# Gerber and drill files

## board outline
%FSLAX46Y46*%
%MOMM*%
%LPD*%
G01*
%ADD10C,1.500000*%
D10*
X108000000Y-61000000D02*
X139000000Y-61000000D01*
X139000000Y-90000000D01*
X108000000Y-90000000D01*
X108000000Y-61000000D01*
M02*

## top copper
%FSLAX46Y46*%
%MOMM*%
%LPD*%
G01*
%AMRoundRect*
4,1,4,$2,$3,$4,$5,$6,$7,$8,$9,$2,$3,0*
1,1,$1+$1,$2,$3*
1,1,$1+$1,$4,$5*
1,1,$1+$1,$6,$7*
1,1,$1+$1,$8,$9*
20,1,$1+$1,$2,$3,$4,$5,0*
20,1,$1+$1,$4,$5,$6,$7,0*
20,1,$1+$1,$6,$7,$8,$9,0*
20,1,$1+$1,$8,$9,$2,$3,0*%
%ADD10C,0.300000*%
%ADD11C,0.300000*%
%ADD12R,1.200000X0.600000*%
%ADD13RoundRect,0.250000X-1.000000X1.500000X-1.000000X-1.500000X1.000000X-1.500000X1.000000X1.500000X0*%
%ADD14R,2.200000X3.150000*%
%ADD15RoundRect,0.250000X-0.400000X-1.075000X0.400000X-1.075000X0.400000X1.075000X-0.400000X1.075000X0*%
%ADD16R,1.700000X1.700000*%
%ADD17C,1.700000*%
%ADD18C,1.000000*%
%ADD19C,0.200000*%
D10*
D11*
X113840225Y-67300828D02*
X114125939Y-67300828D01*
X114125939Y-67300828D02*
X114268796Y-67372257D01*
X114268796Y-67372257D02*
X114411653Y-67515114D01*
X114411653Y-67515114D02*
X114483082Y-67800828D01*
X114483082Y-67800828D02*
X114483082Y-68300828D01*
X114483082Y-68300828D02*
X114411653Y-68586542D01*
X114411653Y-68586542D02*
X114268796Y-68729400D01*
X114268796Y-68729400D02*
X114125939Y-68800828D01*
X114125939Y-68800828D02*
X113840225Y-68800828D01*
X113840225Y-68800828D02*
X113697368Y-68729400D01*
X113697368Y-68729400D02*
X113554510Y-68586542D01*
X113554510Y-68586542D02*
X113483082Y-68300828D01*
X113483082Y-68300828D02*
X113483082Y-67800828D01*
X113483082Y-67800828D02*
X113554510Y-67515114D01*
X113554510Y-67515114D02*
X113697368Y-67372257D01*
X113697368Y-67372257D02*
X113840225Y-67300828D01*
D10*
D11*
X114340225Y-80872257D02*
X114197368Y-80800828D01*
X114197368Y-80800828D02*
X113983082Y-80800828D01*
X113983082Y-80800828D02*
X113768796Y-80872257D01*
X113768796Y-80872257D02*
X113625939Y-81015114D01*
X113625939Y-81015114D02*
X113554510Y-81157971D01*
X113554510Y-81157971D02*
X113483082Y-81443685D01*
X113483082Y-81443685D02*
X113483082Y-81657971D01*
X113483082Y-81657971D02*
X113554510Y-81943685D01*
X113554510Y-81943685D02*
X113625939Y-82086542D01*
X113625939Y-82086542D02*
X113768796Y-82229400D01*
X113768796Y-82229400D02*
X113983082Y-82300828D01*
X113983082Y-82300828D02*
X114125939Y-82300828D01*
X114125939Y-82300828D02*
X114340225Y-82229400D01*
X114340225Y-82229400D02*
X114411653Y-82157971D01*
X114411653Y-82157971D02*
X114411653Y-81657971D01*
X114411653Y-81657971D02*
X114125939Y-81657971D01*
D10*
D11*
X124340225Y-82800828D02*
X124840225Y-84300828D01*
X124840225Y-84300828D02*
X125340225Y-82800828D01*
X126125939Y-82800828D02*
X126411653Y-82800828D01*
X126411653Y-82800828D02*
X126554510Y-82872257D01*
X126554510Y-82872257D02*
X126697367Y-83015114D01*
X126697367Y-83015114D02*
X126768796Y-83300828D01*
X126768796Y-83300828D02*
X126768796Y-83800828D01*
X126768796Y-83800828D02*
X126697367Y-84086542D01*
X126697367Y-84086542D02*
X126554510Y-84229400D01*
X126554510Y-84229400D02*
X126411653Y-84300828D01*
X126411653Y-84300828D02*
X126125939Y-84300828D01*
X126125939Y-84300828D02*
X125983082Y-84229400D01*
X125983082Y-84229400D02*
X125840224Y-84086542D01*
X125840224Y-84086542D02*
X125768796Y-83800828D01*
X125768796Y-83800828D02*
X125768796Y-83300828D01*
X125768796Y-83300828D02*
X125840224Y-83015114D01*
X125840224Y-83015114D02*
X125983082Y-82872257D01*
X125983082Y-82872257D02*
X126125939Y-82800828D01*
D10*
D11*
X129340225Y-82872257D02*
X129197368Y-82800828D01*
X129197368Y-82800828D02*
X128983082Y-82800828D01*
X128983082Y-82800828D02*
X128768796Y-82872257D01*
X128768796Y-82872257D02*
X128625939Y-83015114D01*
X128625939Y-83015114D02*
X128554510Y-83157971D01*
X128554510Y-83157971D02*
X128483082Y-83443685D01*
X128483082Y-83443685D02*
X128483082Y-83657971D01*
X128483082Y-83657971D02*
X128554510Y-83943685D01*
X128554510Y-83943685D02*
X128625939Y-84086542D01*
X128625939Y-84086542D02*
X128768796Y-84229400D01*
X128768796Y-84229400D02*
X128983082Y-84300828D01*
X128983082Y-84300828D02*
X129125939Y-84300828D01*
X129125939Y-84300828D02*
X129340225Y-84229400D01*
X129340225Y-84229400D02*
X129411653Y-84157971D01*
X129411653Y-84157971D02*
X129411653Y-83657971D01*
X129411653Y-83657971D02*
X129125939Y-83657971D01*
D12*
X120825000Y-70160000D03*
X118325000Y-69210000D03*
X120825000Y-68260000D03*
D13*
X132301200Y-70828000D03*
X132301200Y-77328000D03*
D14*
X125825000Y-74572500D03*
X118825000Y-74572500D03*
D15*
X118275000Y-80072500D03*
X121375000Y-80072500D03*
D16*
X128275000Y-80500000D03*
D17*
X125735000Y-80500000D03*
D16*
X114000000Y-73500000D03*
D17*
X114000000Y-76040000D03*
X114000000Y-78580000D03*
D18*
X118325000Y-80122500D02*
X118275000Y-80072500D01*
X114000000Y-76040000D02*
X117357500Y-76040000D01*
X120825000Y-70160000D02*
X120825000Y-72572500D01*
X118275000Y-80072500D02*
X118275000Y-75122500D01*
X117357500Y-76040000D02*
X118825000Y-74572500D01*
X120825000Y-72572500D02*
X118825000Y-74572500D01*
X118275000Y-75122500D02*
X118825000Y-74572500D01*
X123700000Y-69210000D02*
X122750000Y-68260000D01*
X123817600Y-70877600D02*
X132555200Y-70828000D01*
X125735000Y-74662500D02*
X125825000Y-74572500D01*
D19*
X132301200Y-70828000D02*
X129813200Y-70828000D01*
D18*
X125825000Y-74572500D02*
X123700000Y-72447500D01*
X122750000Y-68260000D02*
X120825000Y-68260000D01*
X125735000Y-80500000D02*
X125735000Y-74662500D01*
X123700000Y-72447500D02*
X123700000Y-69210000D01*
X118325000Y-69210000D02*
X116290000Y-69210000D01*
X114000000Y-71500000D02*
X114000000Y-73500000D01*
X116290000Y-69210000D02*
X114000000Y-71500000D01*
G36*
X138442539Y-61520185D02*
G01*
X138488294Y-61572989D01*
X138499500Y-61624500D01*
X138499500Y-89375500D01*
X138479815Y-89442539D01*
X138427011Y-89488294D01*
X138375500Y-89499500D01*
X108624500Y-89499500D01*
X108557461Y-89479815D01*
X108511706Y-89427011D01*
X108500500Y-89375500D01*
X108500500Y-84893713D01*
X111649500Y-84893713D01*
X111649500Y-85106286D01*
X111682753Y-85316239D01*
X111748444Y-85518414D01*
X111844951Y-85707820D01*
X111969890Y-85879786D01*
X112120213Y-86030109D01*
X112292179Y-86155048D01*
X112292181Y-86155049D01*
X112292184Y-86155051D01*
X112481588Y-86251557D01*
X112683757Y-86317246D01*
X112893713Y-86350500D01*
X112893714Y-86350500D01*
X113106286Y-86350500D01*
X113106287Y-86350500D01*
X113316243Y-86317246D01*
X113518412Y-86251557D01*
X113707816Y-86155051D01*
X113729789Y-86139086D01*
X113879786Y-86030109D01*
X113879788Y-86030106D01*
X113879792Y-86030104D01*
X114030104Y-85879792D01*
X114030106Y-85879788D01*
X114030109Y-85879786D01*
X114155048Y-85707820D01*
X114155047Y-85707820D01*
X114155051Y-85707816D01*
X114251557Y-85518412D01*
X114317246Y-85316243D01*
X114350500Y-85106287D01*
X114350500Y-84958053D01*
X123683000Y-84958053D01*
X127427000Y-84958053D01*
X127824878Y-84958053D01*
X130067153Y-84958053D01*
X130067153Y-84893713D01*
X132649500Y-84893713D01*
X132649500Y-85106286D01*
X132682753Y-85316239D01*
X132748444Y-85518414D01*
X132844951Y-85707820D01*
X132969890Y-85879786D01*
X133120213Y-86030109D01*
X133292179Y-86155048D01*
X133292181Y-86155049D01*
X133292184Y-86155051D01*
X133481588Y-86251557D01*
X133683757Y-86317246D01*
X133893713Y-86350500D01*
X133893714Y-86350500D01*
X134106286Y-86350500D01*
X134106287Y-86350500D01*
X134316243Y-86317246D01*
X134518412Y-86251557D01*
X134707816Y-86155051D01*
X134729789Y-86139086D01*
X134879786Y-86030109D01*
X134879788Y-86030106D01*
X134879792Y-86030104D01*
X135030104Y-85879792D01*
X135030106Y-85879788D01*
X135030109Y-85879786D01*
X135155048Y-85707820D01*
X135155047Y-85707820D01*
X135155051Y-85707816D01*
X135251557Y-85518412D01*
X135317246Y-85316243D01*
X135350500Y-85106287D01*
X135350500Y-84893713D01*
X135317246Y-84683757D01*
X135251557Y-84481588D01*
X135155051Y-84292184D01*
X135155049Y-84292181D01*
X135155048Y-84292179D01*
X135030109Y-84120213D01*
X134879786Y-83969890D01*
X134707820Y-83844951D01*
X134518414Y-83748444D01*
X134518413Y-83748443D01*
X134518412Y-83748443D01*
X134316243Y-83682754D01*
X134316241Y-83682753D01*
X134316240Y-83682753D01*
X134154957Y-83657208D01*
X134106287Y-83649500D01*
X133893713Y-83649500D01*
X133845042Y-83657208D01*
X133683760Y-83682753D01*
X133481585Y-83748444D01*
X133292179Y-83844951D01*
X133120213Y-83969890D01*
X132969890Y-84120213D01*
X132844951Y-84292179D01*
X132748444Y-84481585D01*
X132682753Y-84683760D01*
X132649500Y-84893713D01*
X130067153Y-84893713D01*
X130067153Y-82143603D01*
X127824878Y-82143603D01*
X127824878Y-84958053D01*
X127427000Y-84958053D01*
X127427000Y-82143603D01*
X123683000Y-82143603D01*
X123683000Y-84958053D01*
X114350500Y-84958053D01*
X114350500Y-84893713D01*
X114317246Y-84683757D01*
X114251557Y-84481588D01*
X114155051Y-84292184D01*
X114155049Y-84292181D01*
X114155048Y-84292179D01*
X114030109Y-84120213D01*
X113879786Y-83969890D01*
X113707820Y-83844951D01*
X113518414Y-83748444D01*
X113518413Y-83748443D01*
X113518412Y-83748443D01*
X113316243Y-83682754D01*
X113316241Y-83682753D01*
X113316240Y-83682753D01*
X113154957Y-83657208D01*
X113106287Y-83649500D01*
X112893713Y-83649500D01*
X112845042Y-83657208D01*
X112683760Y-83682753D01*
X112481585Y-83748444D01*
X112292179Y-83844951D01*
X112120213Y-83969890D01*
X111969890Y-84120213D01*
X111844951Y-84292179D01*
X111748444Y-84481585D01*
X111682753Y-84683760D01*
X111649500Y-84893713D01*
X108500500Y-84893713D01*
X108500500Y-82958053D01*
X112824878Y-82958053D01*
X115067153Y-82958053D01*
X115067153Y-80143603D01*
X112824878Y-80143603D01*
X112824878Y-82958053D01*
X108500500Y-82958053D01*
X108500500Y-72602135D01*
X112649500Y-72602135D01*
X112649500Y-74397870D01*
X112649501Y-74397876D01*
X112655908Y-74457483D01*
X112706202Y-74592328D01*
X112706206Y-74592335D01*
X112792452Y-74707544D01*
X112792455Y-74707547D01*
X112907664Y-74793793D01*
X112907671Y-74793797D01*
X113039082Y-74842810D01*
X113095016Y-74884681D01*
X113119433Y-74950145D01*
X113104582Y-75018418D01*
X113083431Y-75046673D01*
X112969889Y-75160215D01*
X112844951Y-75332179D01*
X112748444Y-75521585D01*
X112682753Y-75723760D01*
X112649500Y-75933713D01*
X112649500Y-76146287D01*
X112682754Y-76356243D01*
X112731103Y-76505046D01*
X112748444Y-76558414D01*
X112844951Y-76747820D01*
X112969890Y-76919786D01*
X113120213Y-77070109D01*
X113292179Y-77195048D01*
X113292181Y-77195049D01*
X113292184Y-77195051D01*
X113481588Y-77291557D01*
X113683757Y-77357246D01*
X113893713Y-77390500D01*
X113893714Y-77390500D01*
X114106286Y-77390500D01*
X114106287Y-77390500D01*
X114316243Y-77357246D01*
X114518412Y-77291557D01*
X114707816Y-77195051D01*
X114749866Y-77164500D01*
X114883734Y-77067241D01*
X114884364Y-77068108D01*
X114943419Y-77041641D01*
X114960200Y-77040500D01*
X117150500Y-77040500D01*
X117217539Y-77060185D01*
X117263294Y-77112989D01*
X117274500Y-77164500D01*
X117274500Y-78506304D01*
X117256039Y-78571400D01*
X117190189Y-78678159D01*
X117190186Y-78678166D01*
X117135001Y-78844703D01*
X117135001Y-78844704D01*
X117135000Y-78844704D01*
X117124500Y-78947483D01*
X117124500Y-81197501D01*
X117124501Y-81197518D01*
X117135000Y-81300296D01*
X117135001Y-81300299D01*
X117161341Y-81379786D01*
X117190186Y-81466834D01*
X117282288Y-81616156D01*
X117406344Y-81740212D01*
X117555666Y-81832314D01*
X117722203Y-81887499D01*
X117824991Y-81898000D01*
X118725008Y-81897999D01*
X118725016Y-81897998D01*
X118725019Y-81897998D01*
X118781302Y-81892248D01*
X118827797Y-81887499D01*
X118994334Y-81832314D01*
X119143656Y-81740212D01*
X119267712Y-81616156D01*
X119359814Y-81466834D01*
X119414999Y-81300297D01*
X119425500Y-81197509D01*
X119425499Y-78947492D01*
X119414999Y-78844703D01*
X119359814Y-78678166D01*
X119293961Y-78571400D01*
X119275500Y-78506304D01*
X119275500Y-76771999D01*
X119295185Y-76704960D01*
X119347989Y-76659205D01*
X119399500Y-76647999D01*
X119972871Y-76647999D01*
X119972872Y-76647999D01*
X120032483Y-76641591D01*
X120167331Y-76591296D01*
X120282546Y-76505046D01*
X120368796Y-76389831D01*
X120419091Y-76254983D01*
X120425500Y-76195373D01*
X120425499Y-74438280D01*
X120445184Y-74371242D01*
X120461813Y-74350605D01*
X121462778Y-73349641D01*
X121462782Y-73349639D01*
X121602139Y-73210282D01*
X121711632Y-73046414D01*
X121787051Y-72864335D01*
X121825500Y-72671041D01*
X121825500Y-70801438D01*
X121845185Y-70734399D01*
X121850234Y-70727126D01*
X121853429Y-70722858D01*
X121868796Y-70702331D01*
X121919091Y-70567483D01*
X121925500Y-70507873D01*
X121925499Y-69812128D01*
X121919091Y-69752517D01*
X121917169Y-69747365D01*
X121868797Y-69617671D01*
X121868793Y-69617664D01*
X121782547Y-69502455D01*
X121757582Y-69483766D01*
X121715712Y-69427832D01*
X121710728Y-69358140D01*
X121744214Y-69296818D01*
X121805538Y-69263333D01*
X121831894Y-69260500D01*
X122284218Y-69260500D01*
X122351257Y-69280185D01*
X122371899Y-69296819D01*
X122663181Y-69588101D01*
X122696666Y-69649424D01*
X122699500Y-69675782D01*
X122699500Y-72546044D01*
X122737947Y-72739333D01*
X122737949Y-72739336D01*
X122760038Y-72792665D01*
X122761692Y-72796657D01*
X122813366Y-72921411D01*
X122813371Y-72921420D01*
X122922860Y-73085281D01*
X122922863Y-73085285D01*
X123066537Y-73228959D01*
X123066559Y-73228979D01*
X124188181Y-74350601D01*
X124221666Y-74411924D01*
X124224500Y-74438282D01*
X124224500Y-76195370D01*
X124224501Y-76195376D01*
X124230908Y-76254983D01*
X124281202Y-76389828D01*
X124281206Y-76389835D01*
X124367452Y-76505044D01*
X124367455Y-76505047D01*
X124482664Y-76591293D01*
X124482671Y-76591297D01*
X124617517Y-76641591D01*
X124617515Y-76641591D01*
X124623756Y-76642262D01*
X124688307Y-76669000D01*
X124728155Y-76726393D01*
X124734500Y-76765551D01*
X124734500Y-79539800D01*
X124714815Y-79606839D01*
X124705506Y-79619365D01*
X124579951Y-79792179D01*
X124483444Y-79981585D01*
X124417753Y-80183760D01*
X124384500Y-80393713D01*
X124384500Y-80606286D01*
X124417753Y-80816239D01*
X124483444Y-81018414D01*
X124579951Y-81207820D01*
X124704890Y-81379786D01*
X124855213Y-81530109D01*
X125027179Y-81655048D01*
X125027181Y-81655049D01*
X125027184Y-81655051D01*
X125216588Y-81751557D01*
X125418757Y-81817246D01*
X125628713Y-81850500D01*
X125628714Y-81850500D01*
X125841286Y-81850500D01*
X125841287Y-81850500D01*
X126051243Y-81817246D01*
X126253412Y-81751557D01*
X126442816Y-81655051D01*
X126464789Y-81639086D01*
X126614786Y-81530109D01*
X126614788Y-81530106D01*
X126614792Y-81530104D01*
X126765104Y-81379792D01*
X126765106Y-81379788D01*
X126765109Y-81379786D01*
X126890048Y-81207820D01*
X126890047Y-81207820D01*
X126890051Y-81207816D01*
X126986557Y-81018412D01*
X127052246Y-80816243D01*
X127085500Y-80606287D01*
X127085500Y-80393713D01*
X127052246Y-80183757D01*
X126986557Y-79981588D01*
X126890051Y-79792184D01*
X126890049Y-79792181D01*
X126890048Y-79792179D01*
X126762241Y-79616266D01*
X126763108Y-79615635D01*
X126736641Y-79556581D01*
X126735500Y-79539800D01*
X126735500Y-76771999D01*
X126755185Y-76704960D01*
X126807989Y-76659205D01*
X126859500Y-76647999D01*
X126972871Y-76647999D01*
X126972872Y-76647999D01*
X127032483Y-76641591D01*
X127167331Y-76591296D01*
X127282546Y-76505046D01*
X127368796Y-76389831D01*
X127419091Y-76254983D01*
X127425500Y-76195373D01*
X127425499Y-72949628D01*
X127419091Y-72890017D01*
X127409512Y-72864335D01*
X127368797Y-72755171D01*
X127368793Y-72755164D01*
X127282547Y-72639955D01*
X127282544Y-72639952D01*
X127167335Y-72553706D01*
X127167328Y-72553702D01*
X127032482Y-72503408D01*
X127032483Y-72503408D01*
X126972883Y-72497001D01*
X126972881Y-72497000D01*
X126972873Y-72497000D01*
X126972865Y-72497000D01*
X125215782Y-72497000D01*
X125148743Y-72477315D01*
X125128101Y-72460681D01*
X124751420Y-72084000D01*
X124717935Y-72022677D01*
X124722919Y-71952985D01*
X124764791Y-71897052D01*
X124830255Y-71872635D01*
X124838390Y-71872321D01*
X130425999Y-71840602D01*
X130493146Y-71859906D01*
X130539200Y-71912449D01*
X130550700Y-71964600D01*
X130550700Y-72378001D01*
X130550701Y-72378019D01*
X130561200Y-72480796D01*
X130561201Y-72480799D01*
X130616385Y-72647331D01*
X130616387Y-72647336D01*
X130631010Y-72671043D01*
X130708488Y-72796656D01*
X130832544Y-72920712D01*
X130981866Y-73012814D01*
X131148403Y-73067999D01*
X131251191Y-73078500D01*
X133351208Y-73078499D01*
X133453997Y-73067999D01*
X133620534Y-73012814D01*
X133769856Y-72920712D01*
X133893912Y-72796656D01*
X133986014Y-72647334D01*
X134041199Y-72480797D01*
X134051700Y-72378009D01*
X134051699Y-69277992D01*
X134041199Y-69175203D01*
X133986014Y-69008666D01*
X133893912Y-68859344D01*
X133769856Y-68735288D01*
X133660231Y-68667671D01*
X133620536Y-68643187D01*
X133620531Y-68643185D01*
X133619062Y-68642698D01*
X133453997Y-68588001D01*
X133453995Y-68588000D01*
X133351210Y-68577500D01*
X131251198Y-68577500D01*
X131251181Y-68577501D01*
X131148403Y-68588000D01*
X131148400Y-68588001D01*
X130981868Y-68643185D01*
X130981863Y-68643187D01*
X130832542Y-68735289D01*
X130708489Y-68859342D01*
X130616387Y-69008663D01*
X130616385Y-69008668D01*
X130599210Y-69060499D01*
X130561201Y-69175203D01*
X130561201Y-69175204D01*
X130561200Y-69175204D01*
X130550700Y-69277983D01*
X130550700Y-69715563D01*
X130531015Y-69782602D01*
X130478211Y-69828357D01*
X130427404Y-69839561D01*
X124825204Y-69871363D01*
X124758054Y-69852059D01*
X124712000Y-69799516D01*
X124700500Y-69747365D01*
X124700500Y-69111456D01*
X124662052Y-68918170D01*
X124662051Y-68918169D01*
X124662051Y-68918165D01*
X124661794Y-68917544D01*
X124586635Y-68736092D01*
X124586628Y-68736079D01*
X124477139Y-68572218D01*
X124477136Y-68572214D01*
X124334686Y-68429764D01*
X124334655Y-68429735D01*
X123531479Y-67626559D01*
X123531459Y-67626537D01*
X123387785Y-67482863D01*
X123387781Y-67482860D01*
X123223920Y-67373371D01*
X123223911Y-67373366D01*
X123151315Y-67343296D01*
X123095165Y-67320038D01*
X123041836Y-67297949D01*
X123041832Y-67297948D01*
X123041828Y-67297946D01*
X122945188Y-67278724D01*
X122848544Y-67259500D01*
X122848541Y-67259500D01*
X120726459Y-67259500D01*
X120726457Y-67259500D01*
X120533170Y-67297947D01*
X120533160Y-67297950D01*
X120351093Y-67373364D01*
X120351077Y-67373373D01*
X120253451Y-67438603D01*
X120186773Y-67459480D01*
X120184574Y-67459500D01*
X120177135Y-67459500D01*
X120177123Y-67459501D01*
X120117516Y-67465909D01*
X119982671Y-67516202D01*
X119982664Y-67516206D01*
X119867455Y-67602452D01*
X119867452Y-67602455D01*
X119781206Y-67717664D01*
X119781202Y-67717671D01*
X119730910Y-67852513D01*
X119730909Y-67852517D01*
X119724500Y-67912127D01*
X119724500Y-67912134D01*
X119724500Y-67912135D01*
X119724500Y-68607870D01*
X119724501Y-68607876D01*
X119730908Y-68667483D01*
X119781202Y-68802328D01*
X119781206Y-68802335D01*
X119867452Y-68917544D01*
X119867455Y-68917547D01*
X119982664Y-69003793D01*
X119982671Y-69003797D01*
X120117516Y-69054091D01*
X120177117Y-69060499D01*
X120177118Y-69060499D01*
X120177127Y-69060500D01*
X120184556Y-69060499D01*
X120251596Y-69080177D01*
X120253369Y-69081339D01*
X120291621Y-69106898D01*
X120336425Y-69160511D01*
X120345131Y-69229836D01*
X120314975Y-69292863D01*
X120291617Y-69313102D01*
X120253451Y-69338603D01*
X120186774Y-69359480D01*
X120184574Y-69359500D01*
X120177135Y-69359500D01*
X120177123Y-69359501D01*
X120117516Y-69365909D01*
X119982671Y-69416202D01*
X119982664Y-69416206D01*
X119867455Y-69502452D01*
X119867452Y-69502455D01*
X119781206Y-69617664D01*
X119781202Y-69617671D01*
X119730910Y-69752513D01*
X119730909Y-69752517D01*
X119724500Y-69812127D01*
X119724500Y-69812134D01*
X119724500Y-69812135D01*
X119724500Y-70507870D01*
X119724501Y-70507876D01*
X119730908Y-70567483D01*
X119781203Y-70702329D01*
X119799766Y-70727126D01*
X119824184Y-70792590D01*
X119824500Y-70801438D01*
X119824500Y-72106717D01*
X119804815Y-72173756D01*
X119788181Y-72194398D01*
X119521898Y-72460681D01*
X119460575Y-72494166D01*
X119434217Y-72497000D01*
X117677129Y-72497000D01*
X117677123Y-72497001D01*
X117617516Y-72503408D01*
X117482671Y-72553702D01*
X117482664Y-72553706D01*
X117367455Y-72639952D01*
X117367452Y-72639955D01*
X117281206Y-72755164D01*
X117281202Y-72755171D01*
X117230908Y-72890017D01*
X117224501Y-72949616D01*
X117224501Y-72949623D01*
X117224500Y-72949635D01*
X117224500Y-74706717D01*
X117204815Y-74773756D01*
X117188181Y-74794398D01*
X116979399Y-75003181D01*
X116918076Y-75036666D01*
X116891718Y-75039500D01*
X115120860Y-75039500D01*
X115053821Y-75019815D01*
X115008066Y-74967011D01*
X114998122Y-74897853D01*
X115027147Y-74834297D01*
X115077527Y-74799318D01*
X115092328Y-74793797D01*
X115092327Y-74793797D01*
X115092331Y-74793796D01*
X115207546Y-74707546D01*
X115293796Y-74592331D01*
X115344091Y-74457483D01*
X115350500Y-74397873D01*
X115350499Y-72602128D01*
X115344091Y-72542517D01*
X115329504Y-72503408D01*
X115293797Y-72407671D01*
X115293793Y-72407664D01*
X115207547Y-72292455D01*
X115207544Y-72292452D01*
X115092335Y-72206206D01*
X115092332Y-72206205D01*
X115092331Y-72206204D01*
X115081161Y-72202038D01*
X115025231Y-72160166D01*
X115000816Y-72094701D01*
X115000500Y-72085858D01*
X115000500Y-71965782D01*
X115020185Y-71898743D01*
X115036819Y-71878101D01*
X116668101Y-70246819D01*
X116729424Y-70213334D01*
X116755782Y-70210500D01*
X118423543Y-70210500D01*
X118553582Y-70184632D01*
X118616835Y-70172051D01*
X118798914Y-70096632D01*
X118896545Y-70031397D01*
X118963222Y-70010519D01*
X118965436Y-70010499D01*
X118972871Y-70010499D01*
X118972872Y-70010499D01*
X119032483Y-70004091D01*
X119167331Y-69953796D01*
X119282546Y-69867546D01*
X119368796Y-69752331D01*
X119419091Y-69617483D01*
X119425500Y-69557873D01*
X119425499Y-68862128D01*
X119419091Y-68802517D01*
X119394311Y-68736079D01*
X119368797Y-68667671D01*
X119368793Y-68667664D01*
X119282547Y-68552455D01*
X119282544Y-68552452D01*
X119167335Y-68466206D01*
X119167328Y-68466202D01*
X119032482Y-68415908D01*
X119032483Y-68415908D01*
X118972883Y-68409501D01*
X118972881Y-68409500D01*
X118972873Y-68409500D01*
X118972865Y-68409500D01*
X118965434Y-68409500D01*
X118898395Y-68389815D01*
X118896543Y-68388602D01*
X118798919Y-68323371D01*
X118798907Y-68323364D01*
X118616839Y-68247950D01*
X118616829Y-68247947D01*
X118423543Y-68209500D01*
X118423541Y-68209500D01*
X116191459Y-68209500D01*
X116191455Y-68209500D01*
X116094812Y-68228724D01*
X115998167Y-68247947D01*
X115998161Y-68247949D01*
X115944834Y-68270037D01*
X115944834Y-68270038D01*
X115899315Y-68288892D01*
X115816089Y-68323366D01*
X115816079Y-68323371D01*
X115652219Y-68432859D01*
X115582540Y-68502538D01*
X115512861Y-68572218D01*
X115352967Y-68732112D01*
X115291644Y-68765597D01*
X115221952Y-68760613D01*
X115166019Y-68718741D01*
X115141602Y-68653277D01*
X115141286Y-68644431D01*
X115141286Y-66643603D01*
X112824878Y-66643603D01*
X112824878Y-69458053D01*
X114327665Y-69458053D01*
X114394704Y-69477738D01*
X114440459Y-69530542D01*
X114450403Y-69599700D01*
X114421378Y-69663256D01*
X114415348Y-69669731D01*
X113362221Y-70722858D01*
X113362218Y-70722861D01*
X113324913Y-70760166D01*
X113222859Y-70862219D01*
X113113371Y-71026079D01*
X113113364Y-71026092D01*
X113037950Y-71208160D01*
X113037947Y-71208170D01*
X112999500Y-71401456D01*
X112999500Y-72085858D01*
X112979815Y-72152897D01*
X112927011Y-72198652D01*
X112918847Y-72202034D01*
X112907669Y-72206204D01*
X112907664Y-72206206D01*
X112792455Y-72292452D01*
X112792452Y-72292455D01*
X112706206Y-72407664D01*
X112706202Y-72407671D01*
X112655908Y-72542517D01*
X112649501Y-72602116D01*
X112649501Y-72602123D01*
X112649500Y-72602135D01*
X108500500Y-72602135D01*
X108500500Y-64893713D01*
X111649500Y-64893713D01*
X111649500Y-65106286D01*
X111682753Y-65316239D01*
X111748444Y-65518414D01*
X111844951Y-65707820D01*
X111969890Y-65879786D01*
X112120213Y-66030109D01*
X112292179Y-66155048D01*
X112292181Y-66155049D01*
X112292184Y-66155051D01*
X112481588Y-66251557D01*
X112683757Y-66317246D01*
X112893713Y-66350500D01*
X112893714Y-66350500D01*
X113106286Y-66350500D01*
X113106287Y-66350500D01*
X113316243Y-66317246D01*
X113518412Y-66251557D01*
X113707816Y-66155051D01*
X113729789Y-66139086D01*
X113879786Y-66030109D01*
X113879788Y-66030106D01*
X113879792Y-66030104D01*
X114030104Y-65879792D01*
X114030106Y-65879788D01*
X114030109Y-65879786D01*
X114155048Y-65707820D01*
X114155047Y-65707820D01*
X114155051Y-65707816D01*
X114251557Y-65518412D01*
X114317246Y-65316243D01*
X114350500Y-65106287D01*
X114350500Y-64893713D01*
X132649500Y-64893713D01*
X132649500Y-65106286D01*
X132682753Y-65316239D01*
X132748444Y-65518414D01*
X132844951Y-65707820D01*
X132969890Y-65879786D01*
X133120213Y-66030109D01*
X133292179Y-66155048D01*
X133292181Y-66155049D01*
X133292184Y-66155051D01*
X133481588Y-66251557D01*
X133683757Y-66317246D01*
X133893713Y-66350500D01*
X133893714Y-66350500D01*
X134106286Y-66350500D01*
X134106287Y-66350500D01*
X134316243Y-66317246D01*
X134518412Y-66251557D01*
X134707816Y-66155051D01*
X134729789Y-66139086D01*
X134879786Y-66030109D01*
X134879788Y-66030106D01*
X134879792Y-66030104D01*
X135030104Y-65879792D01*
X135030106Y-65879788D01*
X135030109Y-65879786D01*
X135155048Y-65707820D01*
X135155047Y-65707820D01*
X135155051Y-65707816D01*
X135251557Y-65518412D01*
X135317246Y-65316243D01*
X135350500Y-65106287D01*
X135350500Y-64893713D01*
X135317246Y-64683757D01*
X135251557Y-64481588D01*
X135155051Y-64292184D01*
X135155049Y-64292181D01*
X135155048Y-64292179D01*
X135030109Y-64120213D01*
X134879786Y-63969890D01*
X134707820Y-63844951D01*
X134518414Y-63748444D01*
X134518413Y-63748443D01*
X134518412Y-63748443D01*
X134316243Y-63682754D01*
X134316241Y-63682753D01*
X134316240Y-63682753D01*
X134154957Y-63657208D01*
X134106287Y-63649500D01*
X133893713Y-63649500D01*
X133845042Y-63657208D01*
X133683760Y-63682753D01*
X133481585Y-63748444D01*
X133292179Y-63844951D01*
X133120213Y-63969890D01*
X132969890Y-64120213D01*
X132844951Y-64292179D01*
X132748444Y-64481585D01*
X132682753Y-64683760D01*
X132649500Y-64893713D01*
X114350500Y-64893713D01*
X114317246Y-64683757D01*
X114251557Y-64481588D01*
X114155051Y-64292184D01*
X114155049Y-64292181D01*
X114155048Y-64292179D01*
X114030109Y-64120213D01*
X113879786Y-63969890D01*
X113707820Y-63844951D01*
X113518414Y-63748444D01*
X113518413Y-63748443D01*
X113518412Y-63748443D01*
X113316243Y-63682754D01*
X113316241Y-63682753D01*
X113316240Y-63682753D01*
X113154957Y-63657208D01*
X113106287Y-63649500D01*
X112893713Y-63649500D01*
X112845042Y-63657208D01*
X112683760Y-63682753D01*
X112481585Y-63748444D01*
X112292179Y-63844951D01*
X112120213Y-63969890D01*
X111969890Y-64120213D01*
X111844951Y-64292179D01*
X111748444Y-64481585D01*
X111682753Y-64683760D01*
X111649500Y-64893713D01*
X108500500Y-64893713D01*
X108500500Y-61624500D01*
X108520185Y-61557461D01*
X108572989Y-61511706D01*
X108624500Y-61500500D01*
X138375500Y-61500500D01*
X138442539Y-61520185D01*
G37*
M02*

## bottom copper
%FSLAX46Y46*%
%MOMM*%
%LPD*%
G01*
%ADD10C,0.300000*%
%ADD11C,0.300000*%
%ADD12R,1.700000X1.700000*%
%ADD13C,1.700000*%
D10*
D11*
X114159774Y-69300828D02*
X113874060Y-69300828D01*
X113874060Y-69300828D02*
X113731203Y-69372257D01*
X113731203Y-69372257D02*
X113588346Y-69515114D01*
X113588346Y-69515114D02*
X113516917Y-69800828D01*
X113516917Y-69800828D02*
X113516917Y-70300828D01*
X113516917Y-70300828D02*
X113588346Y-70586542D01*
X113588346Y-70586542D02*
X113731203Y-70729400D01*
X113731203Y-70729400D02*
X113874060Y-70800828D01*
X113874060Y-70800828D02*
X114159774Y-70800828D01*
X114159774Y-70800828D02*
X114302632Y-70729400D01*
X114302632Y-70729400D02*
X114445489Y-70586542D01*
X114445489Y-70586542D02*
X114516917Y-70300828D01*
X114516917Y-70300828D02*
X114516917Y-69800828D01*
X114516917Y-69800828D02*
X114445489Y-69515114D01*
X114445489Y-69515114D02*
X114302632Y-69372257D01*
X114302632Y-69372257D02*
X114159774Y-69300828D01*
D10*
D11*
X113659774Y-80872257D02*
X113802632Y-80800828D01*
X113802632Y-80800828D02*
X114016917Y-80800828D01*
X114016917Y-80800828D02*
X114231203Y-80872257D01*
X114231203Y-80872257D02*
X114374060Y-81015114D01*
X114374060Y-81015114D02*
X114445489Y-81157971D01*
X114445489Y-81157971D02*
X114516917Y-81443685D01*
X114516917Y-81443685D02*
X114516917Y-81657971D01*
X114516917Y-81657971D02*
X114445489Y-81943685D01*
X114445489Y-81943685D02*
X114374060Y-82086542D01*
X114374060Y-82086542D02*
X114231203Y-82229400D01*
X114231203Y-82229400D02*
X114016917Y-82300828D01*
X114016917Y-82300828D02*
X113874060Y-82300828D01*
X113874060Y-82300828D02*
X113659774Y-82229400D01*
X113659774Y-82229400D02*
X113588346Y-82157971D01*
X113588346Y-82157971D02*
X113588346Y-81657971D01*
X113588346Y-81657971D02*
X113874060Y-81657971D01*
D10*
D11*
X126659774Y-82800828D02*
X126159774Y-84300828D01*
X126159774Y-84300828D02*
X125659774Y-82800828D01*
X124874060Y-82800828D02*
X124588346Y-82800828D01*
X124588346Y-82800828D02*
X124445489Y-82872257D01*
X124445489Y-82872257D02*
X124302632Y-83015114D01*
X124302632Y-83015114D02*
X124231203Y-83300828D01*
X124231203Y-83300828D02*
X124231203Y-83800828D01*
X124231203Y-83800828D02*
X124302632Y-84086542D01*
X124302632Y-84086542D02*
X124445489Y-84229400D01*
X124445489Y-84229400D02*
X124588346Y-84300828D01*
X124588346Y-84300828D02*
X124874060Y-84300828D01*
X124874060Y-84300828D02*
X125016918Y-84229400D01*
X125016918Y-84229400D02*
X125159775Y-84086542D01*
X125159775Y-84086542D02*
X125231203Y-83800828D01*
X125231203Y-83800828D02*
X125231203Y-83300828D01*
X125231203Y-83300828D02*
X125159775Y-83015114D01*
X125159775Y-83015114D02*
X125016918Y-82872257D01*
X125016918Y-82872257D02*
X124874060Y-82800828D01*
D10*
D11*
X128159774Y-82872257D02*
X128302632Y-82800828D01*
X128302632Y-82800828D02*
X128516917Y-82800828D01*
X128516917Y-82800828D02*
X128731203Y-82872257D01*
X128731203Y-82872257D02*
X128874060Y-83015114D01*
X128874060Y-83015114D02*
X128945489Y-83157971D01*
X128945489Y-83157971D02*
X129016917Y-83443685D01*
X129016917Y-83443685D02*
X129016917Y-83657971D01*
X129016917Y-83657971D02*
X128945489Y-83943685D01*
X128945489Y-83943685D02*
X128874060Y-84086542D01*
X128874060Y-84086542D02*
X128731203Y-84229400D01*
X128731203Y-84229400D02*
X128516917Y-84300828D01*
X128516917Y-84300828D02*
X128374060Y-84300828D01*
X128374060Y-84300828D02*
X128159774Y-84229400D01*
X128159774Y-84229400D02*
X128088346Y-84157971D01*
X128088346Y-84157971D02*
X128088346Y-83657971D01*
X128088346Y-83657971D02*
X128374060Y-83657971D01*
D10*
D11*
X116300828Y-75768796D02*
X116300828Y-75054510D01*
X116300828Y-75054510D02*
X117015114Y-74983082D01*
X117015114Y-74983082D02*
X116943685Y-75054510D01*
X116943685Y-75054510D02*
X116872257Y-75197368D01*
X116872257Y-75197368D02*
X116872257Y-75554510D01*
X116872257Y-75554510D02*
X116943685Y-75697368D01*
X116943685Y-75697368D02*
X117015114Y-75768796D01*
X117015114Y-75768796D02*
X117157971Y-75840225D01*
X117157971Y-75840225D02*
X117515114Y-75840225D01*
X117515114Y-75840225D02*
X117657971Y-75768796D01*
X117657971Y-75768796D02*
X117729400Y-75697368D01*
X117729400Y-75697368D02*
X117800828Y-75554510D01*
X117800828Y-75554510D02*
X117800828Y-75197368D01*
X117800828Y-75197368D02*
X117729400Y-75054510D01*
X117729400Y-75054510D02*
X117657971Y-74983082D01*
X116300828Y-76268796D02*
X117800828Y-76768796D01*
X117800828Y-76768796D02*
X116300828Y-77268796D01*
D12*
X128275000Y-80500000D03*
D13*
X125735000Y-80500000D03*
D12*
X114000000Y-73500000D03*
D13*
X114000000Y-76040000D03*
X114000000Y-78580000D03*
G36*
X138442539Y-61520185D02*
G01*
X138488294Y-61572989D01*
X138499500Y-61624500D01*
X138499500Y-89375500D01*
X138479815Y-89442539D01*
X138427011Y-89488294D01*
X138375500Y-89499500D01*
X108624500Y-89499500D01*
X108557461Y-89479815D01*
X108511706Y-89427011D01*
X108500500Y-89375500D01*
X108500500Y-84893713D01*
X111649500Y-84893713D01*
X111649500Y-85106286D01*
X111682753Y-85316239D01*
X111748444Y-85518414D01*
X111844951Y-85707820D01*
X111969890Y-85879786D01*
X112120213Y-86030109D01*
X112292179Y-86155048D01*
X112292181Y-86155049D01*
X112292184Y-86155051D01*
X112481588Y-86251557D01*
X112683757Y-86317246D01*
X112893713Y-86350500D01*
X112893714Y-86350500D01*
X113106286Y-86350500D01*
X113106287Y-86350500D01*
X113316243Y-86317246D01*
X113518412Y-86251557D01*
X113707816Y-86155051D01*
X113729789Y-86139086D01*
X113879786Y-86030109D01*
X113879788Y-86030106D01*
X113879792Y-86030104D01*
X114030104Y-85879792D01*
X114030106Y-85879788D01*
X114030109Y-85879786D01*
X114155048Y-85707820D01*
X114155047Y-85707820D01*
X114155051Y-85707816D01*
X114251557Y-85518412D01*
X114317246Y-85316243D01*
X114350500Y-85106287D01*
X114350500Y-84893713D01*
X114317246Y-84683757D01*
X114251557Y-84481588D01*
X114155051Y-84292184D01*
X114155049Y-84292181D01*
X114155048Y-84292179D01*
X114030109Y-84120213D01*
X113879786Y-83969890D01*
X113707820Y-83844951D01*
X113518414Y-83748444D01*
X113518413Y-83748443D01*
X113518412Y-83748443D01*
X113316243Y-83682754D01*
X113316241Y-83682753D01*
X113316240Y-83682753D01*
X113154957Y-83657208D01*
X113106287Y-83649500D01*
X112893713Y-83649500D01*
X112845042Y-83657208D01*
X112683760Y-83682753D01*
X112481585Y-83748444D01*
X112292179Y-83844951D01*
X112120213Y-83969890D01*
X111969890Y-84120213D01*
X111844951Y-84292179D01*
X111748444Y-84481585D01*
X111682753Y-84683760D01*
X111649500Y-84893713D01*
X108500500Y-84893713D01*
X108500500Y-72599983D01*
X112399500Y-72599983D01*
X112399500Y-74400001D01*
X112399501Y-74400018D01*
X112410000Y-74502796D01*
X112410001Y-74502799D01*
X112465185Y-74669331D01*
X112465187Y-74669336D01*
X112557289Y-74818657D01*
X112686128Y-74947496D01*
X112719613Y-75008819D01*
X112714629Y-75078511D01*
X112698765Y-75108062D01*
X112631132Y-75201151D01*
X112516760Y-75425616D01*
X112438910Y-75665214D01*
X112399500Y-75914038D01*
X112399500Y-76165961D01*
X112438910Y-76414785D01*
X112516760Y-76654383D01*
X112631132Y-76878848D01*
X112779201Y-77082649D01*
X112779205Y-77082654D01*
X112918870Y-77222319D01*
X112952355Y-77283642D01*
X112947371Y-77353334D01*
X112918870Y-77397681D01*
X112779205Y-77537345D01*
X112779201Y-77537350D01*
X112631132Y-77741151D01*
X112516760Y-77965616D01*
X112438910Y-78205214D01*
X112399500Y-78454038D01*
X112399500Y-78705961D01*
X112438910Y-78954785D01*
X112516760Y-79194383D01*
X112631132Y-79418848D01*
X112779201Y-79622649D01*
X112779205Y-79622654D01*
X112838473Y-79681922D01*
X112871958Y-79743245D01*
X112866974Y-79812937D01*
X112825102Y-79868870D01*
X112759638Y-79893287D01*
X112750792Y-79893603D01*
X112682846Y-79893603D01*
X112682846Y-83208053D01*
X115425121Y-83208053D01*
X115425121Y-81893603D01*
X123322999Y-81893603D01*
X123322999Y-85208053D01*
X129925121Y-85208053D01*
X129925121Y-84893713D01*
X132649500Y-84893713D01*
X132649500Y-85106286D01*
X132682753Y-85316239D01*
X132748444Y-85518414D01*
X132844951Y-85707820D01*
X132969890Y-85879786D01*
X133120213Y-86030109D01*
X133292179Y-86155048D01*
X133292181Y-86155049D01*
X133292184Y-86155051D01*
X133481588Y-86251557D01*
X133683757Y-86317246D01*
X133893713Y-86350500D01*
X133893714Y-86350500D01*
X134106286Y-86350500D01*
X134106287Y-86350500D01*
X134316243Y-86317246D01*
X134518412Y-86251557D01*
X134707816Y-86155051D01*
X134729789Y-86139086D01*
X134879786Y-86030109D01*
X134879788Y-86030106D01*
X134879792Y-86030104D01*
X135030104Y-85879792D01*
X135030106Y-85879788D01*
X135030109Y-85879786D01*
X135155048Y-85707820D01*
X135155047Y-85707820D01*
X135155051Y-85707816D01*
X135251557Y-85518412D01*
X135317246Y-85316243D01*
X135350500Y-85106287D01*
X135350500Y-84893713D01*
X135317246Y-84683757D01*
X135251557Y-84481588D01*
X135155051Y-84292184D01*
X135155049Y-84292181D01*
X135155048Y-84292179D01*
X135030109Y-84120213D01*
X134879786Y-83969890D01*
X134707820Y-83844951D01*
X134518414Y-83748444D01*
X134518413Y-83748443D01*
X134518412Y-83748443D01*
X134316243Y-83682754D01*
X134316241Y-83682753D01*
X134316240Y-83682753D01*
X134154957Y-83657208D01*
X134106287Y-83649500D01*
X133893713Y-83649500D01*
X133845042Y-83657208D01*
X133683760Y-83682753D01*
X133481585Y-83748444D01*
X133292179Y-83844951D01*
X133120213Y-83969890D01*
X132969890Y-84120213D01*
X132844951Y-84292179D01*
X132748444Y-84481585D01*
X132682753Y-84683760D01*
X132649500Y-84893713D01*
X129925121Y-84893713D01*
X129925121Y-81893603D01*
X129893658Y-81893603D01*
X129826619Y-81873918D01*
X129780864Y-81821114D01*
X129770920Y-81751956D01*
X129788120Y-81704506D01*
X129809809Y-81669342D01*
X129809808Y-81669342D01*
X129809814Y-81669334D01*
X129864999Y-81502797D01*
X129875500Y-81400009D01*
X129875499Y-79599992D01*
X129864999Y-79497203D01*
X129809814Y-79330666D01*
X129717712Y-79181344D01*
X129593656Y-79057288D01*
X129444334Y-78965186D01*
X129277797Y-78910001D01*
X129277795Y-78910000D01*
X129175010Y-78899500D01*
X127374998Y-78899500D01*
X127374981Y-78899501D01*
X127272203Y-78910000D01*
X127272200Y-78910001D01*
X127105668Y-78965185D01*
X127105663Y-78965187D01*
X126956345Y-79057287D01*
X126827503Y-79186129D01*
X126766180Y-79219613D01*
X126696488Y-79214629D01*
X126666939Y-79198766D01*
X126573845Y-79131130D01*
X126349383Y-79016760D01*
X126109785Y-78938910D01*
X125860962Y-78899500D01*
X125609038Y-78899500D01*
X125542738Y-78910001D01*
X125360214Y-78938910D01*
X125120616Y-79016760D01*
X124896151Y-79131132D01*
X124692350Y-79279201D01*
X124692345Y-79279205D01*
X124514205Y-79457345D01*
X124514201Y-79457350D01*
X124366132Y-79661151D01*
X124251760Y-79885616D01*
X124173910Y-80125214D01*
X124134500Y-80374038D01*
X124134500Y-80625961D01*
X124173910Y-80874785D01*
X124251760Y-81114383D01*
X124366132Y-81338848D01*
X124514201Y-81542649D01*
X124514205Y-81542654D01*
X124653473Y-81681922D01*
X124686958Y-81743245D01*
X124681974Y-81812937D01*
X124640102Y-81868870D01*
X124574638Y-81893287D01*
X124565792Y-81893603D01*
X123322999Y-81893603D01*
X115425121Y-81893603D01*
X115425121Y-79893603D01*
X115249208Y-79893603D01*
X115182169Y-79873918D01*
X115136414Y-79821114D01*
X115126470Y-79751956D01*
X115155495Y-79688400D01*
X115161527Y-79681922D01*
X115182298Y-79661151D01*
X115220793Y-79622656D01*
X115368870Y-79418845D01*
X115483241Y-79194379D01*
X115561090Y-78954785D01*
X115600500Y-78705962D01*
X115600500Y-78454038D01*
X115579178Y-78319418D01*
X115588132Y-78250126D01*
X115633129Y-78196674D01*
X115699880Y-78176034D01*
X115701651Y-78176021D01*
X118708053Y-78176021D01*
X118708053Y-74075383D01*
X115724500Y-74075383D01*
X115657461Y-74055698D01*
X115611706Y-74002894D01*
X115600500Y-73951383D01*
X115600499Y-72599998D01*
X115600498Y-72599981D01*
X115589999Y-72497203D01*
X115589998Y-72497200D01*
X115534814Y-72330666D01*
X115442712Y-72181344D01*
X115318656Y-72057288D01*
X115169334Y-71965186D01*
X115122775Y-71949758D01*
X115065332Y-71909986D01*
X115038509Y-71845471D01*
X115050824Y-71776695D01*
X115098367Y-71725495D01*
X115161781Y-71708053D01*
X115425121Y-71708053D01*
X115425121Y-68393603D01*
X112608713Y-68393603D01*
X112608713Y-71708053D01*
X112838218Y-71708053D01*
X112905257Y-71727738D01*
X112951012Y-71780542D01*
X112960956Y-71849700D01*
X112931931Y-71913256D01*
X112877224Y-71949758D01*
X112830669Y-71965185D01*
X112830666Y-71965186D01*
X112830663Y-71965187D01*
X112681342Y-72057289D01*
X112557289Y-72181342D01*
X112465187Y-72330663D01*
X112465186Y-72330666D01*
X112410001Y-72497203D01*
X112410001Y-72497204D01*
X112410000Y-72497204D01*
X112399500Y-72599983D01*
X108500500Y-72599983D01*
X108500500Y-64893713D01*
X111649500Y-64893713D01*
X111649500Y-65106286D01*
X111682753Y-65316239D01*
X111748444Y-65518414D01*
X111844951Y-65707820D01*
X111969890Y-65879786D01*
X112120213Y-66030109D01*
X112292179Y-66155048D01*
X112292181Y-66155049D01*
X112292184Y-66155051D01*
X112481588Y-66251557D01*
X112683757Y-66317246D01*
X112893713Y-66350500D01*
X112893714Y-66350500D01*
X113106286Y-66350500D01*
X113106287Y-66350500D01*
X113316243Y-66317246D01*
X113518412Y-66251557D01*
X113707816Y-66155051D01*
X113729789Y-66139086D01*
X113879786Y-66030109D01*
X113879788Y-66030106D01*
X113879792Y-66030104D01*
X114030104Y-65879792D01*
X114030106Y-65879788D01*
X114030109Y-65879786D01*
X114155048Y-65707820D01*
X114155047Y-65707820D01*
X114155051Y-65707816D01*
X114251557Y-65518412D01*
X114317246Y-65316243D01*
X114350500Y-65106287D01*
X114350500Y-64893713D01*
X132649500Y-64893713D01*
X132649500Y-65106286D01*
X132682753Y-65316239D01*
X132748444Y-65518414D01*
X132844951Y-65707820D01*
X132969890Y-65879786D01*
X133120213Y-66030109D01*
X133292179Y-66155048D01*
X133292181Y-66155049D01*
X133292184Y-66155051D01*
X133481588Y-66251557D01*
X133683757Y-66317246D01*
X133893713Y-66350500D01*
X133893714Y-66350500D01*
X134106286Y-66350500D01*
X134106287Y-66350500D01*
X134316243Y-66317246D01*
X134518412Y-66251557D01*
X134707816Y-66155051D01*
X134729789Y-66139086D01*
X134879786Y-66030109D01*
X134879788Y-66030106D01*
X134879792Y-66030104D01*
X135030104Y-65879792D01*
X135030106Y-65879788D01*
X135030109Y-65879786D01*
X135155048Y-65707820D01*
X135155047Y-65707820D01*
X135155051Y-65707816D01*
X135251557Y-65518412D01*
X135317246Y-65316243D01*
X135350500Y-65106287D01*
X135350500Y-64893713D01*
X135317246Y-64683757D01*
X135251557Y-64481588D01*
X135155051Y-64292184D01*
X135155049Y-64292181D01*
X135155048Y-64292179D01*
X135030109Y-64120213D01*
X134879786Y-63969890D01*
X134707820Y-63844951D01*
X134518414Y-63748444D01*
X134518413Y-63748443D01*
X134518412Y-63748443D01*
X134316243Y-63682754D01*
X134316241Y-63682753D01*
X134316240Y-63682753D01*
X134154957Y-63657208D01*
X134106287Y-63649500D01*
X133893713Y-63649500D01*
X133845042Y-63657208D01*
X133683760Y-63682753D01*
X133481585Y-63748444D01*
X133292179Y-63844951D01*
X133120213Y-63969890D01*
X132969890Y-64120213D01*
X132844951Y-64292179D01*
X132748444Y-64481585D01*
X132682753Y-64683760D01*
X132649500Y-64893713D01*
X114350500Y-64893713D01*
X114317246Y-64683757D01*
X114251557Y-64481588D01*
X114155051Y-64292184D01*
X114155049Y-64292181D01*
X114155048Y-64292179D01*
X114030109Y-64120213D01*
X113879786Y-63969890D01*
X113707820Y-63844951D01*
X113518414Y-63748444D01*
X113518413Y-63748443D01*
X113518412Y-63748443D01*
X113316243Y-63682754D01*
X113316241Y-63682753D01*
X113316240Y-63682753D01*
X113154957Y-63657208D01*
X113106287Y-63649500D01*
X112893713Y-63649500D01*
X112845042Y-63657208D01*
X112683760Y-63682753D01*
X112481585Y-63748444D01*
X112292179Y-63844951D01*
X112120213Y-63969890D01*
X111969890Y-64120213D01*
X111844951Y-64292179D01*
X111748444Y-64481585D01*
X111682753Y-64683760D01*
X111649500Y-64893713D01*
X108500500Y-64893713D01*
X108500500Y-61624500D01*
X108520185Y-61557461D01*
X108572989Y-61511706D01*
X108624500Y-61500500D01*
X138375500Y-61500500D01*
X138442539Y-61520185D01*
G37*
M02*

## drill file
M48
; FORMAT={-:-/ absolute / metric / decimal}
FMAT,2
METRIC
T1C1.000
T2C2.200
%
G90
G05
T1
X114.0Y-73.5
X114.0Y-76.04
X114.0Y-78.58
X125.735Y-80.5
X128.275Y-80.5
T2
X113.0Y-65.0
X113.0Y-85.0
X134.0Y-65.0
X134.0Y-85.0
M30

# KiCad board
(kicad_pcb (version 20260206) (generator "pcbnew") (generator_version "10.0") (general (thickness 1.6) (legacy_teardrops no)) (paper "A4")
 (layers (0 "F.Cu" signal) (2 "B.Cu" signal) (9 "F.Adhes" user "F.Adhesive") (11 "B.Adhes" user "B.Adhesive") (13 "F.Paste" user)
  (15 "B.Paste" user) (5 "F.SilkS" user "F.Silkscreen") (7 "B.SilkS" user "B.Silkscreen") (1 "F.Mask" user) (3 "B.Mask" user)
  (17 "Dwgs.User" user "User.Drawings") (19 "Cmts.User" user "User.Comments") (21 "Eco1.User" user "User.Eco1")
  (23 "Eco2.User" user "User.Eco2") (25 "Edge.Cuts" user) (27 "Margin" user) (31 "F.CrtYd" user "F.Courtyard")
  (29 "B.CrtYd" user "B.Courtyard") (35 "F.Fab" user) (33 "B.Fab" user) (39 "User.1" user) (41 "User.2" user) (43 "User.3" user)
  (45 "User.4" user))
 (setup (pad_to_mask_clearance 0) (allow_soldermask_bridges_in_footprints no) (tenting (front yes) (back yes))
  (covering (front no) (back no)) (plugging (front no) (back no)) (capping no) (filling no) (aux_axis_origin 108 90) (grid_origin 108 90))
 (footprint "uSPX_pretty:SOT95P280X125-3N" (layer "F.Cu") (at 119.575 69.21 180)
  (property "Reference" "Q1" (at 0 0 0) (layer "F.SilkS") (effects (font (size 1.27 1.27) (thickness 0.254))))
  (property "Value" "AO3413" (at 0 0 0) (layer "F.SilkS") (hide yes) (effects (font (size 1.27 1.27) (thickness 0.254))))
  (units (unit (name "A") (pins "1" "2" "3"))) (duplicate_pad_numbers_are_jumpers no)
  (pad "1" smd rect (at -1.25 -0.95 270) (size 0.6 1.2) (layers "F.Cu" "F.Mask" "F.Paste") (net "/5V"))
  (pad "2" smd rect (at 1.25 0 270) (size 0.6 1.2) (layers "F.Cu" "F.Mask" "F.Paste") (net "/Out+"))
  (pad "3" smd rect (at -1.25 0.95 270) (size 0.6 1.2) (layers "F.Cu" "F.Mask" "F.Paste") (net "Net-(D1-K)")))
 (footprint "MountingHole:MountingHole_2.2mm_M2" (layer "F.Cu") (at 113 65)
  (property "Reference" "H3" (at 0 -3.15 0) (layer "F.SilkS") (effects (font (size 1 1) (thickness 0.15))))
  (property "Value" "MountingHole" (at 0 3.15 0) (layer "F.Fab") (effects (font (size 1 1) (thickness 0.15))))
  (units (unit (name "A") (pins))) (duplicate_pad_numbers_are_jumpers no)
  (pad "" np_thru_hole circle (at 0 0) (size 2.2 2.2) (drill 2.2) (layers "*.Cu" "*.Mask")))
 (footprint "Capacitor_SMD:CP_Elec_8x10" (layer "F.Cu") (at 132.3012 74.078 -90)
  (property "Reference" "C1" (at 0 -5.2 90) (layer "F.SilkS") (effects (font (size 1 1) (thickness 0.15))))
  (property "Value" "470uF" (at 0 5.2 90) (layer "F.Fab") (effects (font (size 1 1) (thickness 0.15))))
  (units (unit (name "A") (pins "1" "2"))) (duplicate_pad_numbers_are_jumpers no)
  (pad "1" smd roundrect (at -3.25 0 270) (size 3.5 2.5) (layers "F.Cu" "F.Mask" "F.Paste") (roundrect_rratio 0.1) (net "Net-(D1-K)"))
  (pad "2" smd roundrect (at 3.25 0 270) (size 3.5 2.5) (layers "F.Cu" "F.Mask" "F.Paste") (roundrect_rratio 0.1) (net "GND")))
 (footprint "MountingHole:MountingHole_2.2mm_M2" (layer "F.Cu") (at 134 65)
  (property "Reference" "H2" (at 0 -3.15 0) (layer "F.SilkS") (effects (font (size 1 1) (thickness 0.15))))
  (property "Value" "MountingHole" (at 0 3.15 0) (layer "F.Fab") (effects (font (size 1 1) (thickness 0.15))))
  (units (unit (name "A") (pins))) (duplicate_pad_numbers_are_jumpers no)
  (pad "" np_thru_hole circle (at 0 0) (size 2.2 2.2) (drill 2.2) (layers "*.Cu" "*.Mask")))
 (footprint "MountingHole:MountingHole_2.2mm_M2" (layer "F.Cu") (at 134 85)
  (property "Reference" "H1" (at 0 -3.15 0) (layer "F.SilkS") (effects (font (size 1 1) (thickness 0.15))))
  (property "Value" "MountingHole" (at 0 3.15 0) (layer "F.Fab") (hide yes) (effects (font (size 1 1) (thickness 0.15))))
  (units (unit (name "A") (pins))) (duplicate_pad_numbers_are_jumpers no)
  (pad "" np_thru_hole circle (at 0 0) (size 2.2 2.2) (drill 2.2) (layers "*.Cu" "*.Mask")))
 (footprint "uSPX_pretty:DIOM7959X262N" (layer "F.Cu") (at 122.325 74.5725 180)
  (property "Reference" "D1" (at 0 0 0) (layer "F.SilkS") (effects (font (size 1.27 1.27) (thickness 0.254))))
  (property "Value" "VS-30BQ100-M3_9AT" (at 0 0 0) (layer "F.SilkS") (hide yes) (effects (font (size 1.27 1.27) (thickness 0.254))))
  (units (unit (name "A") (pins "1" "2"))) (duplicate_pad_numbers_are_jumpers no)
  (pad "1" smd rect (at -3.5 0 180) (size 2.2 3.15) (layers "F.Cu" "F.Mask" "F.Paste") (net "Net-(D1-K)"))
  (pad "2" smd rect (at 3.5 0 180) (size 2.2 3.15) (layers "F.Cu" "F.Mask" "F.Paste") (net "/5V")))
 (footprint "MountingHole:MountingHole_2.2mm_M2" (layer "F.Cu") (at 113 85)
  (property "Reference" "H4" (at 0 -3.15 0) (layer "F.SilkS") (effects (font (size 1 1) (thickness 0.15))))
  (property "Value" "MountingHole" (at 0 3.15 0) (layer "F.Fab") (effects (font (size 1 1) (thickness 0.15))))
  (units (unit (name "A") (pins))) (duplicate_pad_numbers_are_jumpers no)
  (pad "" np_thru_hole circle (at 0 0) (size 2.2 2.2) (drill 2.2) (layers "*.Cu" "*.Mask")))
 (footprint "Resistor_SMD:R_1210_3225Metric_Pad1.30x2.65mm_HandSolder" (layer "F.Cu") (at 119.825 80.0725)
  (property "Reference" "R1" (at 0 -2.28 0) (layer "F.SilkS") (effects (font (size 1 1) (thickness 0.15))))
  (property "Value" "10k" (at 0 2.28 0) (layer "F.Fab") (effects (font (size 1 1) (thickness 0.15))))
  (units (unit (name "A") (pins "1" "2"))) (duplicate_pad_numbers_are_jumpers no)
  (pad "1" smd roundrect (at -1.55 0) (size 1.3 2.65) (layers "F.Cu" "F.Mask" "F.Paste") (roundrect_rratio 0.192308) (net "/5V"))
  (pad "2" smd roundrect (at 1.55 0) (size 1.3 2.65) (layers "F.Cu" "F.Mask" "F.Paste") (roundrect_rratio 0.192308) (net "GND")))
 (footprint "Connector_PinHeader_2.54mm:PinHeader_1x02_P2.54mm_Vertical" (layer "B.Cu") (at 128.275 80.5 90)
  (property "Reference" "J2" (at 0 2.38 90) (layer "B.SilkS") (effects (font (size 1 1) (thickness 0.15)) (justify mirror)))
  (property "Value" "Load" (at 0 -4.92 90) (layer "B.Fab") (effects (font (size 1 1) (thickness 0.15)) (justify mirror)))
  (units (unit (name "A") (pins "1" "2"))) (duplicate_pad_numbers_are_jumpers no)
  (pad "1" thru_hole rect (at 0 0 90) (size 1.7 1.7) (drill 1) (layers "*.Cu" "*.Mask") (remove_unused_layers no) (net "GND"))
  (pad "2" thru_hole circle (at 0 -2.54 90) (size 1.7 1.7) (drill 1) (layers "*.Cu" "*.Mask") (remove_unused_layers no) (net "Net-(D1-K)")))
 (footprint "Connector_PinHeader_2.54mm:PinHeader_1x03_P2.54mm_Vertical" (layer "B.Cu") (at 114 73.5 180)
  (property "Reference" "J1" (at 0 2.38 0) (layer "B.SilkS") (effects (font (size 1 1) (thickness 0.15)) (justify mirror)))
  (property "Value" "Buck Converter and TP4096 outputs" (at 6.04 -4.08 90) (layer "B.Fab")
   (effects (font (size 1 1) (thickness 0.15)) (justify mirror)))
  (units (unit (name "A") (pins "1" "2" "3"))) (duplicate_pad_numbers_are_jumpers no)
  (pad "1" thru_hole rect (at 0 0 180) (size 1.7 1.7) (drill 1) (layers "*.Cu" "*.Mask") (remove_unused_layers no) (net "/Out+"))
  (pad "2" thru_hole circle (at 0 -2.54 180) (size 1.7 1.7) (drill 1) (layers "*.Cu" "*.Mask") (remove_unused_layers no) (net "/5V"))
  (pad "3" thru_hole circle (at 0 -5.08 180) (size 1.7 1.7) (drill 1) (layers "*.Cu" "*.Mask") (remove_unused_layers no) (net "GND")))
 (gr_rect (start 108 61) (end 139 90) (stroke (width 1.5) (type solid)) (fill no) (layer "Edge.Cuts"))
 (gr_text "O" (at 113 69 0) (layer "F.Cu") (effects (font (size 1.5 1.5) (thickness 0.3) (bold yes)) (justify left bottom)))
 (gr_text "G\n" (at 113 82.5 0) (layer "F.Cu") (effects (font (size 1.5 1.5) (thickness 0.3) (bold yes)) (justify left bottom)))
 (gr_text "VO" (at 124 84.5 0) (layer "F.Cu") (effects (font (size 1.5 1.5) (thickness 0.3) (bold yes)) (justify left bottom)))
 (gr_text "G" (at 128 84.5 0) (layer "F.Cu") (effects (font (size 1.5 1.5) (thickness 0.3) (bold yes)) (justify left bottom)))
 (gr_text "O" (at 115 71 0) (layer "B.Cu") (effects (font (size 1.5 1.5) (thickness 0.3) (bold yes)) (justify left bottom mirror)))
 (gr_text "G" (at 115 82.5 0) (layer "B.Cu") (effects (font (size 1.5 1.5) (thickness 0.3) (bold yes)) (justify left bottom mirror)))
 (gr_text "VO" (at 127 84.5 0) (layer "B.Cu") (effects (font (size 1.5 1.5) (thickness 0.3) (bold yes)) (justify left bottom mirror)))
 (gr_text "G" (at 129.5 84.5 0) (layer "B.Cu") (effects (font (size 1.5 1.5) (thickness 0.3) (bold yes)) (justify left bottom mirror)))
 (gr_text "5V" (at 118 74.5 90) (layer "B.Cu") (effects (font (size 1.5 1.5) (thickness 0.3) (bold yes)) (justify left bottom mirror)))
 (segment (start 118.325 80.1225) (end 118.275 80.0725) (width 1) (layer "F.Cu") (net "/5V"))
 (segment (start 114 76.04) (end 117.3575 76.04) (width 1) (layer "F.Cu") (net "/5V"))
 (segment (start 120.825 70.16) (end 120.825 72.5725) (width 1) (layer "F.Cu") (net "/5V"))
 (segment (start 118.275 80.0725) (end 118.275 75.1225) (width 1) (layer "F.Cu") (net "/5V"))
 (segment (start 117.3575 76.04) (end 118.825 74.5725) (width 1) (layer "F.Cu") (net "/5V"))
 (segment (start 120.825 72.5725) (end 118.825 74.5725) (width 1) (layer "F.Cu") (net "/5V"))
 (segment (start 118.275 75.1225) (end 118.825 74.5725) (width 1) (layer "F.Cu") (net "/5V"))
 (segment (start 123.7 69.21) (end 122.75 68.26) (width 1) (layer "F.Cu") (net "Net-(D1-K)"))
 (segment (start 123.8176 70.8776) (end 132.5552 70.828) (width 1) (layer "F.Cu") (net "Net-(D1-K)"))
 (segment (start 125.735 74.6625) (end 125.825 74.5725) (width 1) (layer "F.Cu") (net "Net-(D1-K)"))
 (segment (start 132.3012 70.828) (end 129.8132 70.828) (width 0.2) (layer "F.Cu") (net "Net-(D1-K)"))
 (segment (start 125.825 74.5725) (end 123.7 72.4475) (width 1) (layer "F.Cu") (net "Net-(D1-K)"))
 (segment (start 122.75 68.26) (end 120.825 68.26) (width 1) (layer "F.Cu") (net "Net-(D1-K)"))
 (segment (start 125.735 80.5) (end 125.735 74.6625) (width 1) (layer "F.Cu") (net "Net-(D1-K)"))
 (segment (start 123.7 72.4475) (end 123.7 69.21) (width 1) (layer "F.Cu") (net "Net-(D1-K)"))
 (segment (start 118.325 69.21) (end 116.29 69.21) (width 1) (layer "F.Cu") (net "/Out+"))
 (segment (start 114 71.5) (end 114 73.5) (width 1) (layer "F.Cu") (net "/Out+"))
 (segment (start 116.29 69.21) (end 114 71.5) (width 1) (layer "F.Cu") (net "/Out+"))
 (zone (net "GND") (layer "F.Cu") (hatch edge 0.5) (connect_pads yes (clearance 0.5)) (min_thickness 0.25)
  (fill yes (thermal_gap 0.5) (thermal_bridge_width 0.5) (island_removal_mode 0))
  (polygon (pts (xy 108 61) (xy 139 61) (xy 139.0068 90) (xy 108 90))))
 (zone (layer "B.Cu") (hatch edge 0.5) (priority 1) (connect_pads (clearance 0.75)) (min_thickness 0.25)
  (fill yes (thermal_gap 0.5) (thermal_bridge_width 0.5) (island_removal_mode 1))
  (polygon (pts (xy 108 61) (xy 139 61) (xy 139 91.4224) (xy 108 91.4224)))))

